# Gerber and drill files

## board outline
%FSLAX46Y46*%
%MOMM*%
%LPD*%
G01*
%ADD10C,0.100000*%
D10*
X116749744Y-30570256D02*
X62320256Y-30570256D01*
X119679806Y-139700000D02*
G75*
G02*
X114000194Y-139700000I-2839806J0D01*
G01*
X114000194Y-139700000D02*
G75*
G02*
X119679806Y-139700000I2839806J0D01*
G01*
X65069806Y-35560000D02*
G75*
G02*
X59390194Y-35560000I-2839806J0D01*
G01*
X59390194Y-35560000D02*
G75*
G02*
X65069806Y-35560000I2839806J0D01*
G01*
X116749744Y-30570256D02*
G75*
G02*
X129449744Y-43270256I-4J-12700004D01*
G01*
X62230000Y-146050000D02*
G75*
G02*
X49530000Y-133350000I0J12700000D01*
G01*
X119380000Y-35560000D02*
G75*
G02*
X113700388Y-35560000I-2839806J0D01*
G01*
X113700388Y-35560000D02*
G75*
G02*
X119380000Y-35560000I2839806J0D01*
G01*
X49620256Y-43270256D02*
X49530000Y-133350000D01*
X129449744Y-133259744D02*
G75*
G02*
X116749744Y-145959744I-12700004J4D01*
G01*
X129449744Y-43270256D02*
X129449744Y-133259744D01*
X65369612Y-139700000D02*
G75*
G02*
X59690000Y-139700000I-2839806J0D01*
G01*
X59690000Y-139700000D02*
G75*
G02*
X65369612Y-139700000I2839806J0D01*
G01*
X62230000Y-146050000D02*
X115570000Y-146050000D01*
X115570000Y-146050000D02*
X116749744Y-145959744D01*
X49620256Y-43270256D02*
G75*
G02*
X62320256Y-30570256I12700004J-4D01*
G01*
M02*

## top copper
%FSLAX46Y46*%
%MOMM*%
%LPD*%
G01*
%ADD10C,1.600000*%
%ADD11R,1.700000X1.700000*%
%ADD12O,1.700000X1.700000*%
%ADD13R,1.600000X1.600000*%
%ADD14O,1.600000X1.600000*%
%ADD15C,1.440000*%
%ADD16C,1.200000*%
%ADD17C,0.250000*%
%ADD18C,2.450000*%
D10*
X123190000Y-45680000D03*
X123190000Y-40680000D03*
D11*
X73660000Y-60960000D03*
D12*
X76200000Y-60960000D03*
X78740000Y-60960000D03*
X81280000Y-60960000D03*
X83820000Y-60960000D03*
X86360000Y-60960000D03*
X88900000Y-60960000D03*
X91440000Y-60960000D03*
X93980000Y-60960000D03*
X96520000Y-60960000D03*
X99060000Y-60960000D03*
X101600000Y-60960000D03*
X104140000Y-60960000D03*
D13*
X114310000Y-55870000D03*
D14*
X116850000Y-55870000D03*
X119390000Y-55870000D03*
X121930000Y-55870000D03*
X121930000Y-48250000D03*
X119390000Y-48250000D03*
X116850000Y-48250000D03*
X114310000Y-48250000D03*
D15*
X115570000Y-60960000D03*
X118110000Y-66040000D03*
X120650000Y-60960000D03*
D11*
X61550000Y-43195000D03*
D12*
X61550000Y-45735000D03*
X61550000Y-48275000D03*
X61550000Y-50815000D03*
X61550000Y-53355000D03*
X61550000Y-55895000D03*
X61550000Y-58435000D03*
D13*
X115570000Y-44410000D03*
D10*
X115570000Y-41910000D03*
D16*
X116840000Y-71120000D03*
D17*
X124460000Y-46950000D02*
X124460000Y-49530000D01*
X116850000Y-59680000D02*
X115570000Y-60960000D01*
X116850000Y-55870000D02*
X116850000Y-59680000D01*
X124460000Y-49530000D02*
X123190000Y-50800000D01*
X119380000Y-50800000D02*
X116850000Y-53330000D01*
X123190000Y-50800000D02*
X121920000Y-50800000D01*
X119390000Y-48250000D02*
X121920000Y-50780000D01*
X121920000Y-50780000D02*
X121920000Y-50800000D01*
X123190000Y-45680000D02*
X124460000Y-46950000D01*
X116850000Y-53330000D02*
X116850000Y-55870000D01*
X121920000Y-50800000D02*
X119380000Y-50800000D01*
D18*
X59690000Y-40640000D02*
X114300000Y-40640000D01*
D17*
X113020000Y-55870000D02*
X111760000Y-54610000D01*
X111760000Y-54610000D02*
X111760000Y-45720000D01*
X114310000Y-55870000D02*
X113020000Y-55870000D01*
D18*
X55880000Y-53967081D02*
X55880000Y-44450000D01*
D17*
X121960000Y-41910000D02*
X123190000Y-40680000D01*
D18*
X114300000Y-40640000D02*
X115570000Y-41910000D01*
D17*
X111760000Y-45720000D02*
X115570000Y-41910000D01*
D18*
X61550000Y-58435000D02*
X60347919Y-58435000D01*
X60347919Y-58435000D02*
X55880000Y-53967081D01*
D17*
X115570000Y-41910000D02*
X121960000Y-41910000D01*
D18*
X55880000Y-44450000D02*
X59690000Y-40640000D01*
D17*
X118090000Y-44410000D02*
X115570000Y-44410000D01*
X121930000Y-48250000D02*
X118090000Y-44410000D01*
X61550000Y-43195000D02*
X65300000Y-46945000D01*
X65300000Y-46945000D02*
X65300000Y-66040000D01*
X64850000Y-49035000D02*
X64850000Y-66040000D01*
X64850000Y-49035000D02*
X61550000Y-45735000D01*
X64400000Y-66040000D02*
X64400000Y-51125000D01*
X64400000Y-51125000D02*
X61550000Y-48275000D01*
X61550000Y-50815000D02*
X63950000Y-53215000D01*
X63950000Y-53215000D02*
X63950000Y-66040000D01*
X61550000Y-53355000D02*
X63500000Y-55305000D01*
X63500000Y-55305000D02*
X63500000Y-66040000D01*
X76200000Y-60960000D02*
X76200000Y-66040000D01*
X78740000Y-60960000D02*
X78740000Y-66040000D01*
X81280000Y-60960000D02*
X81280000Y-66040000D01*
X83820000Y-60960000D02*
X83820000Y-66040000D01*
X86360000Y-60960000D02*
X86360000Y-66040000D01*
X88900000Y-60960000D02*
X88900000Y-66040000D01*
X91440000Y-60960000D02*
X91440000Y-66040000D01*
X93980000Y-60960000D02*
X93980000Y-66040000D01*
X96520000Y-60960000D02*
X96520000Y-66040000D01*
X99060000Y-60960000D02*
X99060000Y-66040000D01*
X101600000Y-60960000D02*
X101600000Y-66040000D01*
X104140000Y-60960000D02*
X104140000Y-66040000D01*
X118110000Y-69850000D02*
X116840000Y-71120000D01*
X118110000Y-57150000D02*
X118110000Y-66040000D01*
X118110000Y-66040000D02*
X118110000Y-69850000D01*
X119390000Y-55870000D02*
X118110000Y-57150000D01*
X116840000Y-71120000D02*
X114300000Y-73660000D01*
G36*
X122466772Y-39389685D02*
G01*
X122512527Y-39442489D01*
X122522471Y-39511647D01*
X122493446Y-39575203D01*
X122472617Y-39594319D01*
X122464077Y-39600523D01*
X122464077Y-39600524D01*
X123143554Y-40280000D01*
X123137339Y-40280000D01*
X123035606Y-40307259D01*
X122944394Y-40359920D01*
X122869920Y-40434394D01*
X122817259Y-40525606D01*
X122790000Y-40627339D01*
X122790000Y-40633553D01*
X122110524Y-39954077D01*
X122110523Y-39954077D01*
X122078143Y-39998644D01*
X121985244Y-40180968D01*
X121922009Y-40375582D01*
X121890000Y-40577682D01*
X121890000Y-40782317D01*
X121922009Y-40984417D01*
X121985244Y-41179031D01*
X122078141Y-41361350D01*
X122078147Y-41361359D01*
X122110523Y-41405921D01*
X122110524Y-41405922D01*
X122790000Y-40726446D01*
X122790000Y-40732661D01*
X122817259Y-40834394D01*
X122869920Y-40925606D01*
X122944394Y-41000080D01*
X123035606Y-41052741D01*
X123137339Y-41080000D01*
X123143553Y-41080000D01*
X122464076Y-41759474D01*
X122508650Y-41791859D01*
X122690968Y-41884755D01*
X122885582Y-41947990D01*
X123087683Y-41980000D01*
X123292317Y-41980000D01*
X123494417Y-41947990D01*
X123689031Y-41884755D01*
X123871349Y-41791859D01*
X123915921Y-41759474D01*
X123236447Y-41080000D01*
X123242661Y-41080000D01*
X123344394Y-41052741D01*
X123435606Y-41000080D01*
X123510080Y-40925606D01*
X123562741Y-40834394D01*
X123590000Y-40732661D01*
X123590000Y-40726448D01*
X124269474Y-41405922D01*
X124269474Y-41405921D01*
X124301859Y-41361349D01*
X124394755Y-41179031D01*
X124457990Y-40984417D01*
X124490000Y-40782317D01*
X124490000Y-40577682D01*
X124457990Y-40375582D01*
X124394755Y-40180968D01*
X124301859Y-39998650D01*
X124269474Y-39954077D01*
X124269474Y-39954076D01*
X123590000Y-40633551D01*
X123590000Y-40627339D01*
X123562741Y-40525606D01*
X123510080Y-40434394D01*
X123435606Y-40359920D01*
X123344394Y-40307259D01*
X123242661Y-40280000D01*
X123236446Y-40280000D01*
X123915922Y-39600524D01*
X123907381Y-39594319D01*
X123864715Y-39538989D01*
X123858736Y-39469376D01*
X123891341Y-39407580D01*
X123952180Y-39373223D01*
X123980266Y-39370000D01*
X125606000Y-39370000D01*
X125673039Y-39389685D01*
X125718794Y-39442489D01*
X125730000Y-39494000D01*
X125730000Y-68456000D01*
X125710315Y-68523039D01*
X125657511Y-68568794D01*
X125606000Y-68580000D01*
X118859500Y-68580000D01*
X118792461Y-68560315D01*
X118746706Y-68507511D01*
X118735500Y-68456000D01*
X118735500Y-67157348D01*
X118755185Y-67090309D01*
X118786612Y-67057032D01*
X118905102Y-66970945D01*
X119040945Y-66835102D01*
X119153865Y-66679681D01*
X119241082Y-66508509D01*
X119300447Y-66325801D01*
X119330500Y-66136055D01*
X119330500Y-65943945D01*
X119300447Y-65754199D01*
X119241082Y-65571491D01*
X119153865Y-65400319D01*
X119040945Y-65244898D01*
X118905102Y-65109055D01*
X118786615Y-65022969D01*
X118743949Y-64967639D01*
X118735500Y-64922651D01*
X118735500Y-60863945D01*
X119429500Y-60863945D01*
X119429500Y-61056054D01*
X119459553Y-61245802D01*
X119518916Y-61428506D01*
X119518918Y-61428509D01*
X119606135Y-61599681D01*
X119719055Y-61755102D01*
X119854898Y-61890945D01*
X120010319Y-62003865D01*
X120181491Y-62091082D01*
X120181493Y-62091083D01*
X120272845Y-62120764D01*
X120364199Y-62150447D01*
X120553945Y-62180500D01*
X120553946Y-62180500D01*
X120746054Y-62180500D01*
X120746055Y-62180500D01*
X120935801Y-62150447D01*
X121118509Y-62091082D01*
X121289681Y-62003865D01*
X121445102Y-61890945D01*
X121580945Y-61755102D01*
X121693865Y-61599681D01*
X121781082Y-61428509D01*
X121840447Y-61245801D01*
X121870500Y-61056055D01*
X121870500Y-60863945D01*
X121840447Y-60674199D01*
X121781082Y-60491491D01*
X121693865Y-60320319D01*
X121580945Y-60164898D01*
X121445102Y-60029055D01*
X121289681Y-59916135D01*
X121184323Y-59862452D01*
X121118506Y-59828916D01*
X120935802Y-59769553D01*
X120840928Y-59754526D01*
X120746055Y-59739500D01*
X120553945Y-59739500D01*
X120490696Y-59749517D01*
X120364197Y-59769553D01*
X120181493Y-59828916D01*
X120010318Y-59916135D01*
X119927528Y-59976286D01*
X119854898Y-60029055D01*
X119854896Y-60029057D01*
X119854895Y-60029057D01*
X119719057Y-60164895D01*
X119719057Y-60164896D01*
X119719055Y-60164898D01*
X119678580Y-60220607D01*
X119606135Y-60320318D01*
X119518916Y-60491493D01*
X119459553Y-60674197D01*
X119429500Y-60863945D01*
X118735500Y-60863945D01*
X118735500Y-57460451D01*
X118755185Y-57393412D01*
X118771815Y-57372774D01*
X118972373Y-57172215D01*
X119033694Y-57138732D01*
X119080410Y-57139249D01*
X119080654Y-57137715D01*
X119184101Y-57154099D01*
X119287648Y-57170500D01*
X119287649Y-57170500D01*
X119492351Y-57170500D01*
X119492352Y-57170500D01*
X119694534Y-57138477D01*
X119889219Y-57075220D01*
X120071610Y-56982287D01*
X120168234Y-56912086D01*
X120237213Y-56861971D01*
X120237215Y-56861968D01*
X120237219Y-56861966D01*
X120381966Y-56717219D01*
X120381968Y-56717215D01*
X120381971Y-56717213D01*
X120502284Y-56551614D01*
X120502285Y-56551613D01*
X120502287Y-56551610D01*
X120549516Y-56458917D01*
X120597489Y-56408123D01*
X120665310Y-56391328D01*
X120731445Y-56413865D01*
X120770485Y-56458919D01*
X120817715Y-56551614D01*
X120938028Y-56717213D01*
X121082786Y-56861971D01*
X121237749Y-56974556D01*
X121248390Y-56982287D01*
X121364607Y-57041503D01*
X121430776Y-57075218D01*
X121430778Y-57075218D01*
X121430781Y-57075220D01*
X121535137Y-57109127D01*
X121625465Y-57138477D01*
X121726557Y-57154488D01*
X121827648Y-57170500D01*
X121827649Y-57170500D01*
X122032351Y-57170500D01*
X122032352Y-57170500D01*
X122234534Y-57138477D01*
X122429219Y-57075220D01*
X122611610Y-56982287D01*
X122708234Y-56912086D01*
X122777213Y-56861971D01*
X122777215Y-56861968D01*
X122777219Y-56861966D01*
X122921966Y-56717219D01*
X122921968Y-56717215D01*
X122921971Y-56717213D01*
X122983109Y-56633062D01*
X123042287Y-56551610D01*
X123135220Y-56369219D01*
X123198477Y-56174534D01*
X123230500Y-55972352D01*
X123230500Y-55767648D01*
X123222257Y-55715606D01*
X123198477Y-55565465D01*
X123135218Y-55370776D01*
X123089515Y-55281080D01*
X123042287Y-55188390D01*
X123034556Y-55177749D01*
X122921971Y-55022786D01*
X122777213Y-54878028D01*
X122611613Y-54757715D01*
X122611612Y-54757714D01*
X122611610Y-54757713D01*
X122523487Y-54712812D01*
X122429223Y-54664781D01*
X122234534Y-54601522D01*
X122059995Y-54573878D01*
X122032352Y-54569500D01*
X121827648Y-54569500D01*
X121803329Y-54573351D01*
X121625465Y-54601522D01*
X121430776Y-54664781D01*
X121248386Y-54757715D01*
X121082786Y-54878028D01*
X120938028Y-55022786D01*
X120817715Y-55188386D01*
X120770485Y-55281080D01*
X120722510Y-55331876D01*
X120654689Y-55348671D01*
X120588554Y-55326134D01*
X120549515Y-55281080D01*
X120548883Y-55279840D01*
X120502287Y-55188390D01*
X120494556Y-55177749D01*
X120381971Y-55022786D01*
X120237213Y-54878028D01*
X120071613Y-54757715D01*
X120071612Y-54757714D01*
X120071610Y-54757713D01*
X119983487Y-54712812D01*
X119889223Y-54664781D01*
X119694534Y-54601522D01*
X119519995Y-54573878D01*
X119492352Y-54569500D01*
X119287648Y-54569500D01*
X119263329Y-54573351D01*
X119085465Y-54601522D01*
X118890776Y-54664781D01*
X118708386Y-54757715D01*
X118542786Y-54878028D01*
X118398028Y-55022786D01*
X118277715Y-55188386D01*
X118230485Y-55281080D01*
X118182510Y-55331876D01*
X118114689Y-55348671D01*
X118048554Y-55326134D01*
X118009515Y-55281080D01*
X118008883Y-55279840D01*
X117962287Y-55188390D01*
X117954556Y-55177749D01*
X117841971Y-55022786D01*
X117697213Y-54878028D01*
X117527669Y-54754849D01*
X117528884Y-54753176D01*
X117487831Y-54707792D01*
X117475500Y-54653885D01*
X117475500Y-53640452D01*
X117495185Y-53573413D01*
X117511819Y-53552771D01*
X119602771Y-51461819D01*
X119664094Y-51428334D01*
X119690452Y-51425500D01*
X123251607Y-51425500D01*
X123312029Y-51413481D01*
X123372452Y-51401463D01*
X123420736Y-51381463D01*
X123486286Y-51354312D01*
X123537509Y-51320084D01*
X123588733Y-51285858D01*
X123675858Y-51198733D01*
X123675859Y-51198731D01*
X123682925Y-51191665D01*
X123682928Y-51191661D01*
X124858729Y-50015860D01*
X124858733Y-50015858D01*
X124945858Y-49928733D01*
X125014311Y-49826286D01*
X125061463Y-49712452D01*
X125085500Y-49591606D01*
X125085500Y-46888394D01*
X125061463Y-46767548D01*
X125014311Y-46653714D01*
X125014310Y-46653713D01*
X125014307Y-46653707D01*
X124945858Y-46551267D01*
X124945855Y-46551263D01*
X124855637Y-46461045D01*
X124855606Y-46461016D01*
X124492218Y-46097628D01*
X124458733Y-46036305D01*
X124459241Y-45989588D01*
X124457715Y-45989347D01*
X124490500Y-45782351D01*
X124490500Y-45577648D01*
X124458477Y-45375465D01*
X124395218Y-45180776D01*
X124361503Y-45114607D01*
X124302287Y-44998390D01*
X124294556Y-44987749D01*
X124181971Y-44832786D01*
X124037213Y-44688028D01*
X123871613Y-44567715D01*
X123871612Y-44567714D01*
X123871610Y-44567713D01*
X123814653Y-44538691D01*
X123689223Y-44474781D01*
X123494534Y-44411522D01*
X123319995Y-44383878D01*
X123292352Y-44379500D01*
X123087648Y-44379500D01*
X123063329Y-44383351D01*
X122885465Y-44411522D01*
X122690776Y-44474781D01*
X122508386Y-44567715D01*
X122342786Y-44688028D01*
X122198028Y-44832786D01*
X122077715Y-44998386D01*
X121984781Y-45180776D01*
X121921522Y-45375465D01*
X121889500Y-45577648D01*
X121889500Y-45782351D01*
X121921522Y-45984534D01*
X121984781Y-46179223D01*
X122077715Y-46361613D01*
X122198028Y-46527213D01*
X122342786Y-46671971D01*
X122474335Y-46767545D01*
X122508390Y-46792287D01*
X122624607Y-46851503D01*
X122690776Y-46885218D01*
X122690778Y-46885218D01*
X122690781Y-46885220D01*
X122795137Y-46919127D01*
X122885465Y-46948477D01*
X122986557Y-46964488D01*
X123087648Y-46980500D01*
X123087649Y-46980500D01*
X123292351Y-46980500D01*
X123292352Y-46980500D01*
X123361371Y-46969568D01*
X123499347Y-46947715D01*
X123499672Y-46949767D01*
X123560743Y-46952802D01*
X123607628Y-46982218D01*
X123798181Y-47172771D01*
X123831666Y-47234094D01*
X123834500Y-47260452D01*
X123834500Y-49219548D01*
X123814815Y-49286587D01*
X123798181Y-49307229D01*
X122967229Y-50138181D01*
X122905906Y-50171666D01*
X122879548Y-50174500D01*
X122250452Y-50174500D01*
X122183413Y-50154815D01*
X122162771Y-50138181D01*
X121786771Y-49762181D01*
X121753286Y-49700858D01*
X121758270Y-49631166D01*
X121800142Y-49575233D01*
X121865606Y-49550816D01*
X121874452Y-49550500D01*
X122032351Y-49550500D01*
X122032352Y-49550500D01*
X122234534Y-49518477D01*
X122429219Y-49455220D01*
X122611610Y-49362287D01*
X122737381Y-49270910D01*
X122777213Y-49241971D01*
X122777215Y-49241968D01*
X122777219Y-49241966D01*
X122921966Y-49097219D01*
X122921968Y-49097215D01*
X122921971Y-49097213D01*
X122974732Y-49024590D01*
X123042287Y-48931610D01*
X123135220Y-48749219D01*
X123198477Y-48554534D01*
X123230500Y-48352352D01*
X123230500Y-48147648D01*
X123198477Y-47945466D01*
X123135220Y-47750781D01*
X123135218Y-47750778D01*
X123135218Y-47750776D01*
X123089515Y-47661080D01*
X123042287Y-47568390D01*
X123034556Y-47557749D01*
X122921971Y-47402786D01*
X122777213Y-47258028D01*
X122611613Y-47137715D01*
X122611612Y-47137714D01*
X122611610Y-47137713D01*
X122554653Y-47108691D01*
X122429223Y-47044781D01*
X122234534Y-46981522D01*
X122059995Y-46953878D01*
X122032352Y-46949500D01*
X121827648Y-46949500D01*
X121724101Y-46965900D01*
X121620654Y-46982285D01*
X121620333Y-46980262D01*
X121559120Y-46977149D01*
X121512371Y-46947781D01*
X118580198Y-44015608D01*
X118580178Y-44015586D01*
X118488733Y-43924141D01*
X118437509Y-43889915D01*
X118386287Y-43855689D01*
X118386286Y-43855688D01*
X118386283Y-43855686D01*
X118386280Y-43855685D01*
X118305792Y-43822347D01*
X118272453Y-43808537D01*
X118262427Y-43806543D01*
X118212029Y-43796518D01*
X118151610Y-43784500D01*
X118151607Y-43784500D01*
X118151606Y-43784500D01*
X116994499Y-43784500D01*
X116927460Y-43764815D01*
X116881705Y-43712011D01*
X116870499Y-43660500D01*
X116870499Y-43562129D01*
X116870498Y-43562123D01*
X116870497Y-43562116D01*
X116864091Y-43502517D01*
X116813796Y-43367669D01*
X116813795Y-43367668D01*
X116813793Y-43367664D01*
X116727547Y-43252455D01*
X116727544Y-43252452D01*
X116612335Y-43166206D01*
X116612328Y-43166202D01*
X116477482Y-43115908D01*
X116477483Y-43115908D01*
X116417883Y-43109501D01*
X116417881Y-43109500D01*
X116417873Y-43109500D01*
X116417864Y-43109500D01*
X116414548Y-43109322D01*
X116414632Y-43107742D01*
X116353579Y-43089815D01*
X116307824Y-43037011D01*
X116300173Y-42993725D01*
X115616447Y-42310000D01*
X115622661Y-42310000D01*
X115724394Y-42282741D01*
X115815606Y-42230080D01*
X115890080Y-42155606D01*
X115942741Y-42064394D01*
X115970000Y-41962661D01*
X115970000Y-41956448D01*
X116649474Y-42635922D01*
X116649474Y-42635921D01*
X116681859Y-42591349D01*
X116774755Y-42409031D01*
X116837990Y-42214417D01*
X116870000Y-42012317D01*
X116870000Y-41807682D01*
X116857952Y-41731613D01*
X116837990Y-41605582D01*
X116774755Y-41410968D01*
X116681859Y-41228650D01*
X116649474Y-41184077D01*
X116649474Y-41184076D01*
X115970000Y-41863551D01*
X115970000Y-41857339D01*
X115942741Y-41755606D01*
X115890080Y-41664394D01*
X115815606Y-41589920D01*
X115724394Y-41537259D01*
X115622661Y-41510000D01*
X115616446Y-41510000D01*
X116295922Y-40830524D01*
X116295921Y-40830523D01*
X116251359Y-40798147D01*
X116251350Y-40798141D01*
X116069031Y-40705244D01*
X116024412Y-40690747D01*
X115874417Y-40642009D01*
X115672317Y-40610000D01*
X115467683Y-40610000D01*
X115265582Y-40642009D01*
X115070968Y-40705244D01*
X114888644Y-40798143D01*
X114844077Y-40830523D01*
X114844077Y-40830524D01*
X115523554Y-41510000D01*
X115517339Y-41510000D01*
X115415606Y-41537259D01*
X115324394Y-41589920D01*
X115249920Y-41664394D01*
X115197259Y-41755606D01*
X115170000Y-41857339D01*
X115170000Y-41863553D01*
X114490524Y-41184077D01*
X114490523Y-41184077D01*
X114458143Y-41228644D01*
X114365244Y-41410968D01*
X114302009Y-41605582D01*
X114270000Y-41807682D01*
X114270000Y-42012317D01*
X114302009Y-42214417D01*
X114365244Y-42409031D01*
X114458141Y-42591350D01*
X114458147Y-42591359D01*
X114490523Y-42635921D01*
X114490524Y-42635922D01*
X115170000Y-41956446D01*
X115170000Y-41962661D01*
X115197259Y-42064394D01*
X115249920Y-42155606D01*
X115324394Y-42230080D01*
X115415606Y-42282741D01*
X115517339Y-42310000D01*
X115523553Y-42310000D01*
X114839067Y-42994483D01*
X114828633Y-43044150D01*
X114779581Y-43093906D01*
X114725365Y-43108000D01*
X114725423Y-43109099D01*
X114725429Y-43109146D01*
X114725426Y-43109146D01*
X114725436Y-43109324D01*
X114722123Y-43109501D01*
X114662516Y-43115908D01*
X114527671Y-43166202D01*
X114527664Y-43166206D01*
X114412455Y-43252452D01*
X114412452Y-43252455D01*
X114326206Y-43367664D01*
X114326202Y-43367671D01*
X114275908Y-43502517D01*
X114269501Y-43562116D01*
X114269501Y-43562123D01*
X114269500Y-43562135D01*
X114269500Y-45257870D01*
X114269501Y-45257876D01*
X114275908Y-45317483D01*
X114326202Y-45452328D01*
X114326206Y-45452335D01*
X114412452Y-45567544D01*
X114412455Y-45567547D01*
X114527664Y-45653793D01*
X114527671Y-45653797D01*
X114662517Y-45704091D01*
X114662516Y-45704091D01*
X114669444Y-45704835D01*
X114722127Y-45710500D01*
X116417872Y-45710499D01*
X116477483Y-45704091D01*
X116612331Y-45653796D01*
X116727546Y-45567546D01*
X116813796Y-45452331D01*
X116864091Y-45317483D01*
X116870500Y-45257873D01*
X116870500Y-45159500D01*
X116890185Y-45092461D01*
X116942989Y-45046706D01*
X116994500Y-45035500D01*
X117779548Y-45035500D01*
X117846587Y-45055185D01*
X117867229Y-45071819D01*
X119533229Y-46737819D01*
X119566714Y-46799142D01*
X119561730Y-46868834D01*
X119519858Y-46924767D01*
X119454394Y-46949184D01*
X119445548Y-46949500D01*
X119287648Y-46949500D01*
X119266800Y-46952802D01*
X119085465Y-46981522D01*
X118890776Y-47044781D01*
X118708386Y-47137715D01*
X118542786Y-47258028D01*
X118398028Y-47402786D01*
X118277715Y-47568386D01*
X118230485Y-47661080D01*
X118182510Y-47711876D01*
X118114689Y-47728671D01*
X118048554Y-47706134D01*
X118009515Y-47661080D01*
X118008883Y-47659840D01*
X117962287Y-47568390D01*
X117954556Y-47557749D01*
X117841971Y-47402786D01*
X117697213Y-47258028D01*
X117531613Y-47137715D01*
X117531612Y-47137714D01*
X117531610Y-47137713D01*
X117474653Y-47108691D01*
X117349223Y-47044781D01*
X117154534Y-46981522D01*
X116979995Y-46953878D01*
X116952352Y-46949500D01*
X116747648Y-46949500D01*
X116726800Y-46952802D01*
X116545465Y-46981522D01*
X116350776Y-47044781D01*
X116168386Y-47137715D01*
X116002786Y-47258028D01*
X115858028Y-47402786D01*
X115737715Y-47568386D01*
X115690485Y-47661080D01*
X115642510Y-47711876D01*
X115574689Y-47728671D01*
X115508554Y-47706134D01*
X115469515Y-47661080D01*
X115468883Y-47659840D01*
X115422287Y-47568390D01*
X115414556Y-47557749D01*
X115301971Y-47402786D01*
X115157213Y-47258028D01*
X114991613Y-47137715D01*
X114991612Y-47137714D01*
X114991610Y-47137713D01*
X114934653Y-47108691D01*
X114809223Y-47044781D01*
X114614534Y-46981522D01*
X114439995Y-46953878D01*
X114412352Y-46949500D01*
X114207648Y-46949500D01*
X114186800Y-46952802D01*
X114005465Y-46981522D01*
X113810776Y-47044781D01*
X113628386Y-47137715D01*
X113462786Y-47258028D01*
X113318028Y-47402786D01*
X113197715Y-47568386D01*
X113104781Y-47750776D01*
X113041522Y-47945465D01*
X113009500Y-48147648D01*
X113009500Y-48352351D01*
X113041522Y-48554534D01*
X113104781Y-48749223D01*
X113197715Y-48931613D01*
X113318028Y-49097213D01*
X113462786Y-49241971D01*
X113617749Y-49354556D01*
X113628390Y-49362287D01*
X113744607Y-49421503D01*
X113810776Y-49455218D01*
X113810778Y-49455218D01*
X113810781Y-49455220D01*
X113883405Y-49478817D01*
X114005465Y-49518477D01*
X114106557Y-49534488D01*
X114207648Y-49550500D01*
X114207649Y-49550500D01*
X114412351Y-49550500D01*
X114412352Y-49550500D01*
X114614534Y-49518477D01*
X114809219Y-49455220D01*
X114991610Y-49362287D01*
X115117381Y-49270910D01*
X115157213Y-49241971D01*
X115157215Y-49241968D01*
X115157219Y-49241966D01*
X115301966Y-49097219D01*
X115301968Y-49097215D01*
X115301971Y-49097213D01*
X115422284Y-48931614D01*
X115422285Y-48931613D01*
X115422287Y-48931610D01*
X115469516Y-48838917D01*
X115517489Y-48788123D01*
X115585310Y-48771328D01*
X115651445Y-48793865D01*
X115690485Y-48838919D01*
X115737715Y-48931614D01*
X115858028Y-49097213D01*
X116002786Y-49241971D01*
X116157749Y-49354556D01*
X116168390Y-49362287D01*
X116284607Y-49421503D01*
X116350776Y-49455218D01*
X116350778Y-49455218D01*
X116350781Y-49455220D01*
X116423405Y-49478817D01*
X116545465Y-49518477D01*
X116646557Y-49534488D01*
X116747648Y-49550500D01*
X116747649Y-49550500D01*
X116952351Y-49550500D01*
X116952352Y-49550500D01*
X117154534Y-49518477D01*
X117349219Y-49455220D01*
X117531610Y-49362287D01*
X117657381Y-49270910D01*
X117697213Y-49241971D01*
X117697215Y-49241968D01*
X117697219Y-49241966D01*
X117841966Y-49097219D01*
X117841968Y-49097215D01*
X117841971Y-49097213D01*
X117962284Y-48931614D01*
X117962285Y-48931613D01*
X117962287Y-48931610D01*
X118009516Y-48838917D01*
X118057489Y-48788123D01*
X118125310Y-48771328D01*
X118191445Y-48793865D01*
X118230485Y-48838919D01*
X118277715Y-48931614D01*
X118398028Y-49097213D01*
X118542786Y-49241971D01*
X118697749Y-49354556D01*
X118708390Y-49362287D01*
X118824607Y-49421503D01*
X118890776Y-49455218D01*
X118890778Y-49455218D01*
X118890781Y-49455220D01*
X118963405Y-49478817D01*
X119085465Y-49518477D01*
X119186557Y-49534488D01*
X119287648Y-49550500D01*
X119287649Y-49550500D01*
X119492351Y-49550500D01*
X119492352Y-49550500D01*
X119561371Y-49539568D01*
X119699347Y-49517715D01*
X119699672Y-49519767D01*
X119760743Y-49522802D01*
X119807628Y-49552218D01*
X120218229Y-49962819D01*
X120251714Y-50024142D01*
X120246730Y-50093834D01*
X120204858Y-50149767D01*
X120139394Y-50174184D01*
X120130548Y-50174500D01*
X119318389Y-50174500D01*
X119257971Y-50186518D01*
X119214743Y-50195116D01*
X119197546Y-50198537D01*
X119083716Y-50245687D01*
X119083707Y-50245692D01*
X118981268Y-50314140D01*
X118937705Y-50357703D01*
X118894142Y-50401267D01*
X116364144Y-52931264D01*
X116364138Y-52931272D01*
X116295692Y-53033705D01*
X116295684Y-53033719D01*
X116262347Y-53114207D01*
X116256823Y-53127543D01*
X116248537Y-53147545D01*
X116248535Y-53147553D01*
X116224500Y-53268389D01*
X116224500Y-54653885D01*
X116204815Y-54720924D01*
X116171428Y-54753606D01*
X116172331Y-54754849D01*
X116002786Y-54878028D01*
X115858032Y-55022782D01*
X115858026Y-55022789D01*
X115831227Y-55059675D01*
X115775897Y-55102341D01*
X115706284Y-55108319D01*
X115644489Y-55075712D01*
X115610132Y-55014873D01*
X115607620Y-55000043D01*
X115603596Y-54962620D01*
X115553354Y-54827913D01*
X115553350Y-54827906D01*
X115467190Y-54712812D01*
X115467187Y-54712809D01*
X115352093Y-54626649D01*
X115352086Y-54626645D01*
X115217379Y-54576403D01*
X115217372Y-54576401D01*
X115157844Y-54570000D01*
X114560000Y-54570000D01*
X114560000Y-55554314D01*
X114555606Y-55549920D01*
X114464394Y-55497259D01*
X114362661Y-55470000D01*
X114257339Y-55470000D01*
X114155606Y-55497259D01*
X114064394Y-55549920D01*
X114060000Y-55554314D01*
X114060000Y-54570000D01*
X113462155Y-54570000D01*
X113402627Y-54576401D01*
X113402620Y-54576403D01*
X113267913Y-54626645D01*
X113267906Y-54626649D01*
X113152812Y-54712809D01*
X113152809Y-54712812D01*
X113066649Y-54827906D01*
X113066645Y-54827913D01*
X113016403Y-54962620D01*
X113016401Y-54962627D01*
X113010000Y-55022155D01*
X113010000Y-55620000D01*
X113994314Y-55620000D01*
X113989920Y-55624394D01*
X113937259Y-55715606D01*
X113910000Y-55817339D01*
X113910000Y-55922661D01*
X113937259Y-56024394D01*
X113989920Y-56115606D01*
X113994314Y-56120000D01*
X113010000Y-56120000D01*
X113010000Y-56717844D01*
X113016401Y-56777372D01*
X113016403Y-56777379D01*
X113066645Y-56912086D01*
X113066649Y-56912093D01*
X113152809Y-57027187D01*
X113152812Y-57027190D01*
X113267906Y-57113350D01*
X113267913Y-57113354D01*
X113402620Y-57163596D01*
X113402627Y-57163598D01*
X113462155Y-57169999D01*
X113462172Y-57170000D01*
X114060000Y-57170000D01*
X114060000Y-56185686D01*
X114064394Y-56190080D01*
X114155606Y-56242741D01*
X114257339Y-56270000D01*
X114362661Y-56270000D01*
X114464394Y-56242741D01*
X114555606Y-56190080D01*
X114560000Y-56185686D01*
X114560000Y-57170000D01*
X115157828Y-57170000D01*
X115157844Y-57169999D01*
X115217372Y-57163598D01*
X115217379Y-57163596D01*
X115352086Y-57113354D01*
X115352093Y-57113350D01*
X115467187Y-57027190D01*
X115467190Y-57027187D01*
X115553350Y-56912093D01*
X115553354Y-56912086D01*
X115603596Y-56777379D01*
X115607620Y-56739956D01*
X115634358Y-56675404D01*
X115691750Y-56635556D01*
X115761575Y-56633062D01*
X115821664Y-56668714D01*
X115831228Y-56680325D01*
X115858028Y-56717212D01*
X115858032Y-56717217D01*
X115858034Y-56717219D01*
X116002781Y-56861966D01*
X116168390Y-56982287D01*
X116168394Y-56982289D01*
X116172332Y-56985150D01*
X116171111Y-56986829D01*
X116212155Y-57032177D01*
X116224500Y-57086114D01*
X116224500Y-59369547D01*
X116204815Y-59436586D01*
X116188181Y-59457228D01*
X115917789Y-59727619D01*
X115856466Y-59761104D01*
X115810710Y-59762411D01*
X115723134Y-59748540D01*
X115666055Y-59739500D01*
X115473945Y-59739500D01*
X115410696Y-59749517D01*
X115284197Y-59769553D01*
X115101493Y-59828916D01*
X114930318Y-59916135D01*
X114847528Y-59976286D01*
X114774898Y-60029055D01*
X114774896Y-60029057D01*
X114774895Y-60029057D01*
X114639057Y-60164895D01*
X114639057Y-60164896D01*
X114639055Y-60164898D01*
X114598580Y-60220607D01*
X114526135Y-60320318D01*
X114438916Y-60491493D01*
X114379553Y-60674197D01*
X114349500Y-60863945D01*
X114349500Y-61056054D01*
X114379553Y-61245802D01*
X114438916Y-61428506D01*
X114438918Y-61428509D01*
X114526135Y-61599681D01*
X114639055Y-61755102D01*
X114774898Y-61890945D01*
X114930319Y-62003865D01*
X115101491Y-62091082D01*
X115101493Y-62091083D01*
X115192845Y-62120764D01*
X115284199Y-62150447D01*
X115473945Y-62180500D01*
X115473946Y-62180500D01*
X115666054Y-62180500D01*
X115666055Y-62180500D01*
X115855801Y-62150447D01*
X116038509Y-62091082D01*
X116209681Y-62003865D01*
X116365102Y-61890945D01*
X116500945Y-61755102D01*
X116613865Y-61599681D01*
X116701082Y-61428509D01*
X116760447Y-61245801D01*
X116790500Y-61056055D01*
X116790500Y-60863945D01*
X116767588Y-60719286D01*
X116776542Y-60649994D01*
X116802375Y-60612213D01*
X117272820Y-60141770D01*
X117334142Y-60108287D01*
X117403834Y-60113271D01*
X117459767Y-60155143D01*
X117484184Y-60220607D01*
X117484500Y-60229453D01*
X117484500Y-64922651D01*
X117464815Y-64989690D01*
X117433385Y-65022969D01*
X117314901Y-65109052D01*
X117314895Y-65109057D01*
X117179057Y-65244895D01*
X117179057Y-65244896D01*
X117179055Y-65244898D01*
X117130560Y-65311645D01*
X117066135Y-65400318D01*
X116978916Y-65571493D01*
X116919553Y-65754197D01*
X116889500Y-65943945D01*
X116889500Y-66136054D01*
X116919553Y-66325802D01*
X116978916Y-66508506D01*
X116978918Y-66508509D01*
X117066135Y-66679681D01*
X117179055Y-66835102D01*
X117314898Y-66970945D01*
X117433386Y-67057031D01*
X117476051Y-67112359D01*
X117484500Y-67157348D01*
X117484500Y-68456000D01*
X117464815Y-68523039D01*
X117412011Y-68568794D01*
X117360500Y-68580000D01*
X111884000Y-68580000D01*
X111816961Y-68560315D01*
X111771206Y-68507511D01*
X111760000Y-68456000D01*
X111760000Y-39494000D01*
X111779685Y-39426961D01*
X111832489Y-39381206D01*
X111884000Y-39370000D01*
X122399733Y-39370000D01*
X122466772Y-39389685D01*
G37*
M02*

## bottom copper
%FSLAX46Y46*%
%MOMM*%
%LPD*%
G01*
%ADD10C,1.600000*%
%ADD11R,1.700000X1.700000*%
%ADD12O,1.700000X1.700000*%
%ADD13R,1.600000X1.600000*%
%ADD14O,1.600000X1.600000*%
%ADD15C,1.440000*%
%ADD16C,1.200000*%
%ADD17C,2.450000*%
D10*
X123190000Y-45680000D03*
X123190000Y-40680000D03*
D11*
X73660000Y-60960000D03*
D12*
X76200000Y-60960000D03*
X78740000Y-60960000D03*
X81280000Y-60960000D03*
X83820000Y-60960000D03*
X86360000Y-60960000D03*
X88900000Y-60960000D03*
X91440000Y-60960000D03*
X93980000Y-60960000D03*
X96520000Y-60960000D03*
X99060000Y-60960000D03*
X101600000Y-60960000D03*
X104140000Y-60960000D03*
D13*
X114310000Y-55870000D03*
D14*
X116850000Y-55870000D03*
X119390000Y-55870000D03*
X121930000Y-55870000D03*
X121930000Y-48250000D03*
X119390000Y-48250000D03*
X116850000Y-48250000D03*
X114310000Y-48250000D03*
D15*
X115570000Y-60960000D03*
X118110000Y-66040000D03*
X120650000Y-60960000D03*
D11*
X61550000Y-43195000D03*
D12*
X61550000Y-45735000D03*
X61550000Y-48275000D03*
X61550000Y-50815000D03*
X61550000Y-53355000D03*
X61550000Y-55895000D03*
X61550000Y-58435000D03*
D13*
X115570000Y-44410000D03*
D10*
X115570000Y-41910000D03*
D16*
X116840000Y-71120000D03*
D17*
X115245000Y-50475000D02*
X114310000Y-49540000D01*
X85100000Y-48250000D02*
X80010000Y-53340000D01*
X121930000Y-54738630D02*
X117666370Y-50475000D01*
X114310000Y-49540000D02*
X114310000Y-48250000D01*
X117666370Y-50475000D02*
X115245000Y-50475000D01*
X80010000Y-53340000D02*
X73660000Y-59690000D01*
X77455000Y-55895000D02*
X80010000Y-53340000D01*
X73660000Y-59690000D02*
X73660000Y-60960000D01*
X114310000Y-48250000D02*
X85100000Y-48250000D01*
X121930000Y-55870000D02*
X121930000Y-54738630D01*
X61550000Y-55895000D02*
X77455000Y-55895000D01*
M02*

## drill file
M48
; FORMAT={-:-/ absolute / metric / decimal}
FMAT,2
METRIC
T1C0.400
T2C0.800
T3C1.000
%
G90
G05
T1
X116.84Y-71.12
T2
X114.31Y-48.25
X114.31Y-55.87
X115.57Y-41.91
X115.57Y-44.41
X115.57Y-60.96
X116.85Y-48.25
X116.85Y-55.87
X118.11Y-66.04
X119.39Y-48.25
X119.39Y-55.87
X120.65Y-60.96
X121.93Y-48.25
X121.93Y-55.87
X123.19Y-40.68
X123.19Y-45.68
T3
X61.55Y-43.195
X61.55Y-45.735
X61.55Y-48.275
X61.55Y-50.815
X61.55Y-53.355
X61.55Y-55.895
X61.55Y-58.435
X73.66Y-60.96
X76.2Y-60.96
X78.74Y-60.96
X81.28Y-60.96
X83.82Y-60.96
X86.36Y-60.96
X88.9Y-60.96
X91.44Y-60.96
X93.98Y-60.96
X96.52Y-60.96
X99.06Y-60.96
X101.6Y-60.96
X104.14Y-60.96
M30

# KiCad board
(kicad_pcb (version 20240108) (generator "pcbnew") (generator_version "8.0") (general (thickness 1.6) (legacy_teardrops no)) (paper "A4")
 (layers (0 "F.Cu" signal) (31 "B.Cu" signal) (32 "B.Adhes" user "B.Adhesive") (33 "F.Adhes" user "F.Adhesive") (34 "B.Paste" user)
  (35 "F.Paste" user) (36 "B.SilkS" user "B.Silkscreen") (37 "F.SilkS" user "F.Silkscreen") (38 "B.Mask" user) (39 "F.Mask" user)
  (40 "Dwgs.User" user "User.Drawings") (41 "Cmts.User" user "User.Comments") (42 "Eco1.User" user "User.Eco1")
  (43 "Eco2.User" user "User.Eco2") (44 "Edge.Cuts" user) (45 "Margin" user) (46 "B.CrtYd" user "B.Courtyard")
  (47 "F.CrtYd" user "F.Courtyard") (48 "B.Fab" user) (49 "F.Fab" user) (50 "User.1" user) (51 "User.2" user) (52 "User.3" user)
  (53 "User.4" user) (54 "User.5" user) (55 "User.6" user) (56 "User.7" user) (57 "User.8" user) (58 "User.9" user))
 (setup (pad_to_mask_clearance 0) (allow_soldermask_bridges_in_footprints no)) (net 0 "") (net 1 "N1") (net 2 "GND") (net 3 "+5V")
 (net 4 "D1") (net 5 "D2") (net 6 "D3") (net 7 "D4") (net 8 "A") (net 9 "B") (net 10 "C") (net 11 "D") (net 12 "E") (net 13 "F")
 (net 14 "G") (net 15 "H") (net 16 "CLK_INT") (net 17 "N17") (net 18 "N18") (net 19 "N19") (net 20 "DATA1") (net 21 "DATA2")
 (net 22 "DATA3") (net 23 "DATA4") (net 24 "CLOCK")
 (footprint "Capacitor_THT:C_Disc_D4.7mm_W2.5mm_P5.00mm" (layer "F.Cu") (at 123.19 45.68 90)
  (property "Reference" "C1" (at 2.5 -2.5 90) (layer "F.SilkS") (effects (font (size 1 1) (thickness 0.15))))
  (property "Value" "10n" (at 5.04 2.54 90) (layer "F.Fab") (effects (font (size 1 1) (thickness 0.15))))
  (pad "1" thru_hole circle (at 0 0 90) (size 1.6 1.6) (drill 0.8) (layers "*.Cu" "*.Mask") (remove_unused_layers no) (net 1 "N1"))
  (pad "2" thru_hole circle (at 5 0 90) (size 1.6 1.6) (drill 0.8) (layers "*.Cu" "*.Mask") (remove_unused_layers no) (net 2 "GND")))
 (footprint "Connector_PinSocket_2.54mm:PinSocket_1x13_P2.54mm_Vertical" (layer "F.Cu") (at 73.66 60.96 90)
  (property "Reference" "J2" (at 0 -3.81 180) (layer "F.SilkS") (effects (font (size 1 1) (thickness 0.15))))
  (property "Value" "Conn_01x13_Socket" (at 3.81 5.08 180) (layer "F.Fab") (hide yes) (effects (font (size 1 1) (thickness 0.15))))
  (pad "1" thru_hole rect (at 0 0 90) (size 1.7 1.7) (drill 1) (layers "*.Cu" "*.Mask") (remove_unused_layers no) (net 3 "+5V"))
  (pad "2" thru_hole oval (at 0 2.54 90) (size 1.7 1.7) (drill 1) (layers "*.Cu" "*.Mask") (remove_unused_layers no) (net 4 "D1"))
  (pad "3" thru_hole oval (at 0 5.08 90) (size 1.7 1.7) (drill 1) (layers "*.Cu" "*.Mask") (remove_unused_layers no) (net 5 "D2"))
  (pad "4" thru_hole oval (at 0 7.62 90) (size 1.7 1.7) (drill 1) (layers "*.Cu" "*.Mask") (remove_unused_layers no) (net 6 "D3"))
  (pad "5" thru_hole oval (at 0 10.16 90) (size 1.7 1.7) (drill 1) (layers "*.Cu" "*.Mask") (remove_unused_layers no) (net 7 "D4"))
  (pad "6" thru_hole oval (at 0 12.7 90) (size 1.7 1.7) (drill 1) (layers "*.Cu" "*.Mask") (remove_unused_layers no) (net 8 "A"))
  (pad "7" thru_hole oval (at 0 15.24 90) (size 1.7 1.7) (drill 1) (layers "*.Cu" "*.Mask") (remove_unused_layers no) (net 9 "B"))
  (pad "8" thru_hole oval (at 0 17.78 90) (size 1.7 1.7) (drill 1) (layers "*.Cu" "*.Mask") (remove_unused_layers no) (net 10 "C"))
  (pad "9" thru_hole oval (at 0 20.32 90) (size 1.7 1.7) (drill 1) (layers "*.Cu" "*.Mask") (remove_unused_layers no) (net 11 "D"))
  (pad "10" thru_hole oval (at 0 22.86 90) (size 1.7 1.7) (drill 1) (layers "*.Cu" "*.Mask") (remove_unused_layers no) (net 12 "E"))
  (pad "11" thru_hole oval (at 0 25.4 90) (size 1.7 1.7) (drill 1) (layers "*.Cu" "*.Mask") (remove_unused_layers no) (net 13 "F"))
  (pad "12" thru_hole oval (at 0 27.94 90) (size 1.7 1.7) (drill 1) (layers "*.Cu" "*.Mask") (remove_unused_layers no) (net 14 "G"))
  (pad "13" thru_hole oval (at 0 30.48 90) (size 1.7 1.7) (drill 1) (layers "*.Cu" "*.Mask") (remove_unused_layers no) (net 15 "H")))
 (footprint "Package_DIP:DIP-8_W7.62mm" (layer "F.Cu") (at 114.31 55.87 90)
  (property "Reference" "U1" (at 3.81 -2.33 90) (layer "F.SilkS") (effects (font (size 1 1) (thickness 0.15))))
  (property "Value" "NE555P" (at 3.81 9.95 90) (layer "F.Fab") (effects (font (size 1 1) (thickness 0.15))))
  (pad "1" thru_hole rect (at 0 0 90) (size 1.6 1.6) (drill 0.8) (layers "*.Cu" "*.Mask") (remove_unused_layers no) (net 2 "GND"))
  (pad "2" thru_hole oval (at 0 2.54 90) (size 1.6 1.6) (drill 0.8) (layers "*.Cu" "*.Mask") (remove_unused_layers no) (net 1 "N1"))
  (pad "3" thru_hole oval (at 0 5.08 90) (size 1.6 1.6) (drill 0.8) (layers "*.Cu" "*.Mask") (remove_unused_layers no) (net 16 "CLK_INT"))
  (pad "4" thru_hole oval (at 0 7.62 90) (size 1.6 1.6) (drill 0.8) (layers "*.Cu" "*.Mask") (remove_unused_layers no) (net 3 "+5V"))
  (pad "5" thru_hole oval (at 7.62 7.62 90) (size 1.6 1.6) (drill 0.8) (layers "*.Cu" "*.Mask") (remove_unused_layers no) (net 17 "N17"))
  (pad "6" thru_hole oval (at 7.62 5.08 90) (size 1.6 1.6) (drill 0.8) (layers "*.Cu" "*.Mask") (remove_unused_layers no) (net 1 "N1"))
  (pad "7" thru_hole oval (at 7.62 2.54 90) (size 1.6 1.6) (drill 0.8) (layers "*.Cu" "*.Mask") (remove_unused_layers no) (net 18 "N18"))
  (pad "8" thru_hole oval (at 7.62 0 90) (size 1.6 1.6) (drill 0.8) (layers "*.Cu" "*.Mask") (remove_unused_layers no) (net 3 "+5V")))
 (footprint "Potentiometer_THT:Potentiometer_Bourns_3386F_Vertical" (layer "F.Cu") (at 115.57 60.96 -90)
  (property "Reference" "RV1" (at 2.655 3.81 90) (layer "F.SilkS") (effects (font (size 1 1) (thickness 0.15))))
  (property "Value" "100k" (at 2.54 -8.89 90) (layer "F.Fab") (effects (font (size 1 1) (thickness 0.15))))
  (pad "1" thru_hole circle (at 0 0 270) (size 1.44 1.44) (drill 0.8) (layers "*.Cu" "*.Mask") (remove_unused_layers no) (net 1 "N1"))
  (pad "2" thru_hole circle (at 5.08 -2.54 270) (size 1.44 1.44) (drill 0.8) (layers "*.Cu" "*.Mask") (remove_unused_layers no)
   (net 16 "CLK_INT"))
  (pad "3" thru_hole circle (at 0 -5.08 270) (size 1.44 1.44) (drill 0.8) (layers "*.Cu" "*.Mask") (remove_unused_layers no) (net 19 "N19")))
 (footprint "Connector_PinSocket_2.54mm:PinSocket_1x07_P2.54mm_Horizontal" (layer "F.Cu") (at 61.55 43.195)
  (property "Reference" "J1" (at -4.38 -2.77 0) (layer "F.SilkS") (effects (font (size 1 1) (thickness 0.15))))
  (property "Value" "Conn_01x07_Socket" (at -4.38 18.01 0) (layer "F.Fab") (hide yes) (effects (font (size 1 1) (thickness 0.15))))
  (pad "1" thru_hole rect (at 0 0) (size 1.7 1.7) (drill 1) (layers "*.Cu" "*.Mask") (remove_unused_layers no) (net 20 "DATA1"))
  (pad "2" thru_hole oval (at 0 2.54) (size 1.7 1.7) (drill 1) (layers "*.Cu" "*.Mask") (remove_unused_layers no) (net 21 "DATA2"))
  (pad "3" thru_hole oval (at 0 5.08) (size 1.7 1.7) (drill 1) (layers "*.Cu" "*.Mask") (remove_unused_layers no) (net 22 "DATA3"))
  (pad "4" thru_hole oval (at 0 7.62) (size 1.7 1.7) (drill 1) (layers "*.Cu" "*.Mask") (remove_unused_layers no) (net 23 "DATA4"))
  (pad "5" thru_hole oval (at 0 10.16) (size 1.7 1.7) (drill 1) (layers "*.Cu" "*.Mask") (remove_unused_layers no) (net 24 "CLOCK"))
  (pad "6" thru_hole oval (at 0 12.7) (size 1.7 1.7) (drill 1) (layers "*.Cu" "*.Mask") (remove_unused_layers no) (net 3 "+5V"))
  (pad "7" thru_hole oval (at 0 15.24) (size 1.7 1.7) (drill 1) (layers "*.Cu" "*.Mask") (remove_unused_layers no) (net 2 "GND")))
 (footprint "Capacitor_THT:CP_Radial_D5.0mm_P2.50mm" (layer "F.Cu") (at 115.57 44.41 90)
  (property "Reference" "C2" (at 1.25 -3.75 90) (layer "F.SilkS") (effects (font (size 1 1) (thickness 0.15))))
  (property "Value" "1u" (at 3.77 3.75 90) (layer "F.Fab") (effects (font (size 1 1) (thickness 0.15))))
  (pad "1" thru_hole rect (at 0 0 90) (size 1.6 1.6) (drill 0.8) (layers "*.Cu" "*.Mask") (remove_unused_layers no) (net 17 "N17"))
  (pad "2" thru_hole circle (at 2.5 0 90) (size 1.6 1.6) (drill 0.8) (layers "*.Cu" "*.Mask") (remove_unused_layers no) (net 2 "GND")))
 (gr_line (start 116.749744 30.570256) (end 62.320256 30.570256) (stroke (width 0.1) (type default)) (layer "Edge.Cuts"))
 (gr_circle (center 116.84 139.7) (end 119.38 140.97) (stroke (width 0.1) (type default)) (fill none) (layer "Edge.Cuts"))
 (gr_circle (center 62.23 35.56) (end 64.77 36.83) (stroke (width 0.1) (type default)) (fill none) (layer "Edge.Cuts"))
 (gr_arc (start 116.749744 30.570256) (mid 125.73 34.29) (end 129.449744 43.270256) (stroke (width 0.1) (type default)) (layer "Edge.Cuts"))
 (gr_arc (start 62.23 146.05) (mid 53.249744 142.330256) (end 49.53 133.35) (stroke (width 0.1) (type default)) (layer "Edge.Cuts"))
 (gr_circle (center 116.540194 35.56) (end 119.080194 36.83) (stroke (width 0.1) (type default)) (fill none) (layer "Edge.Cuts"))
 (gr_line (start 49.620256 43.270256) (end 49.53 133.35) (stroke (width 0.1) (type default)) (layer "Edge.Cuts"))
 (gr_arc (start 129.449744 133.259744) (mid 125.73 142.24) (end 116.749744 145.959744) (stroke (width 0.1) (type default))
  (layer "Edge.Cuts"))
 (gr_line (start 129.449744 43.270256) (end 129.449744 133.259744) (stroke (width 0.1) (type default)) (layer "Edge.Cuts"))
 (gr_circle (center 62.529806 139.7) (end 65.069806 140.97) (stroke (width 0.1) (type default)) (fill none) (layer "Edge.Cuts"))
 (gr_line (start 62.23 146.05) (end 115.57 146.05) (stroke (width 0.1) (type default)) (layer "Edge.Cuts"))
 (gr_line (start 115.57 146.05) (end 116.749744 145.959744) (stroke (width 0.1) (type default)) (layer "Edge.Cuts"))
 (gr_arc (start 49.620256 43.270256) (mid 53.34 34.29) (end 62.320256 30.570256) (stroke (width 0.1) (type default)) (layer "Edge.Cuts"))
 (segment (start 124.46 46.95) (end 124.46 49.53) (width 0.25) (layer "F.Cu") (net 1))
 (segment (start 116.85 59.68) (end 115.57 60.96) (width 0.25) (layer "F.Cu") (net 1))
 (segment (start 116.85 55.87) (end 116.85 59.68) (width 0.25) (layer "F.Cu") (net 1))
 (segment (start 124.46 49.53) (end 123.19 50.8) (width 0.25) (layer "F.Cu") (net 1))
 (segment (start 119.38 50.8) (end 116.85 53.33) (width 0.25) (layer "F.Cu") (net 1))
 (segment (start 123.19 50.8) (end 121.92 50.8) (width 0.25) (layer "F.Cu") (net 1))
 (segment (start 119.39 48.25) (end 121.92 50.78) (width 0.25) (layer "F.Cu") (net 1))
 (segment (start 121.92 50.78) (end 121.92 50.8) (width 0.25) (layer "F.Cu") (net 1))
 (segment (start 123.19 45.68) (end 124.46 46.95) (width 0.25) (layer "F.Cu") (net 1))
 (segment (start 116.85 53.33) (end 116.85 55.87) (width 0.25) (layer "F.Cu") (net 1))
 (segment (start 121.92 50.8) (end 119.38 50.8) (width 0.25) (layer "F.Cu") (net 1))
 (segment (start 59.69 40.64) (end 114.3 40.64) (width 2.45) (layer "F.Cu") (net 2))
 (segment (start 113.02 55.87) (end 111.76 54.61) (width 0.25) (layer "F.Cu") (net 2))
 (segment (start 111.76 54.61) (end 111.76 45.72) (width 0.25) (layer "F.Cu") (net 2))
 (segment (start 114.31 55.87) (end 113.02 55.87) (width 0.25) (layer "F.Cu") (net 2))
 (segment (start 55.88 53.967081) (end 55.88 44.45) (width 2.45) (layer "F.Cu") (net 2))
 (segment (start 121.96 41.91) (end 123.19 40.68) (width 0.25) (layer "F.Cu") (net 2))
 (segment (start 114.3 40.64) (end 115.57 41.91) (width 2.45) (layer "F.Cu") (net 2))
 (segment (start 111.76 45.72) (end 115.57 41.91) (width 0.25) (layer "F.Cu") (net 2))
 (segment (start 61.55 58.435) (end 60.347919 58.435) (width 2.45) (layer "F.Cu") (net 2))
 (segment (start 60.347919 58.435) (end 55.88 53.967081) (width 2.45) (layer "F.Cu") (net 2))
 (segment (start 115.57 41.91) (end 121.96 41.91) (width 0.25) (layer "F.Cu") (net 2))
 (segment (start 55.88 44.45) (end 59.69 40.64) (width 2.45) (layer "F.Cu") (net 2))
 (segment (start 118.09 44.41) (end 115.57 44.41) (width 0.25) (layer "F.Cu") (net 17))
 (segment (start 121.93 48.25) (end 118.09 44.41) (width 0.25) (layer "F.Cu") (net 17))
 (segment (start 61.55 43.195) (end 65.3 46.945) (width 0.25) (layer "F.Cu") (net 20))
 (segment (start 65.3 46.945) (end 65.3 66.04) (width 0.25) (layer "F.Cu") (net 20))
 (segment (start 64.85 49.035) (end 64.85 66.04) (width 0.25) (layer "F.Cu") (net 21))
 (segment (start 64.85 49.035) (end 61.55 45.735) (width 0.25) (layer "F.Cu") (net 21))
 (segment (start 64.4 66.04) (end 64.4 51.125) (width 0.25) (layer "F.Cu") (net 22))
 (segment (start 64.4 51.125) (end 61.55 48.275) (width 0.25) (layer "F.Cu") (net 22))
 (segment (start 61.55 50.815) (end 63.95 53.215) (width 0.25) (layer "F.Cu") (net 23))
 (segment (start 63.95 53.215) (end 63.95 66.04) (width 0.25) (layer "F.Cu") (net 23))
 (segment (start 61.55 53.355) (end 63.5 55.305) (width 0.25) (layer "F.Cu") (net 24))
 (segment (start 63.5 55.305) (end 63.5 66.04) (width 0.25) (layer "F.Cu") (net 24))
 (segment (start 115.245 50.475) (end 114.31 49.54) (width 2.45) (layer "B.Cu") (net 3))
 (segment (start 85.1 48.25) (end 80.01 53.34) (width 2.45) (layer "B.Cu") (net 3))
 (segment (start 121.93 54.73863) (end 117.66637 50.475) (width 2.45) (layer "B.Cu") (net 3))
 (segment (start 114.31 49.54) (end 114.31 48.25) (width 2.45) (layer "B.Cu") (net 3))
 (segment (start 117.66637 50.475) (end 115.245 50.475) (width 2.45) (layer "B.Cu") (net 3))
 (segment (start 80.01 53.34) (end 73.66 59.69) (width 2.45) (layer "B.Cu") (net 3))
 (segment (start 77.455 55.895) (end 80.01 53.34) (width 2.45) (layer "B.Cu") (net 3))
 (segment (start 73.66 59.69) (end 73.66 60.96) (width 2.45) (layer "B.Cu") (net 3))
 (segment (start 114.31 48.25) (end 85.1 48.25) (width 2.45) (layer "B.Cu") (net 3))
 (segment (start 121.93 55.87) (end 121.93 54.73863) (width 2.45) (layer "B.Cu") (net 3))
 (segment (start 61.55 55.895) (end 77.455 55.895) (width 2.45) (layer "B.Cu") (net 3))
 (segment (start 76.2 60.96) (end 76.2 66.04) (width 0.25) (layer "F.Cu") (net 4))
 (segment (start 78.74 60.96) (end 78.74 66.04) (width 0.25) (layer "F.Cu") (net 5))
 (segment (start 81.28 60.96) (end 81.28 66.04) (width 0.25) (layer "F.Cu") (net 6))
 (segment (start 83.82 60.96) (end 83.82 66.04) (width 0.25) (layer "F.Cu") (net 7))
 (segment (start 86.36 60.96) (end 86.36 66.04) (width 0.25) (layer "F.Cu") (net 8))
 (segment (start 88.9 60.96) (end 88.9 66.04) (width 0.25) (layer "F.Cu") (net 9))
 (segment (start 91.44 60.96) (end 91.44 66.04) (width 0.25) (layer "F.Cu") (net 10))
 (segment (start 93.98 60.96) (end 93.98 66.04) (width 0.25) (layer "F.Cu") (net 11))
 (segment (start 96.52 60.96) (end 96.52 66.04) (width 0.25) (layer "F.Cu") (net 12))
 (segment (start 99.06 60.96) (end 99.06 66.04) (width 0.25) (layer "F.Cu") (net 13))
 (segment (start 101.6 60.96) (end 101.6 66.04) (width 0.25) (layer "F.Cu") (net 14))
 (segment (start 104.14 60.96) (end 104.14 66.04) (width 0.25) (layer "F.Cu") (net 15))
 (segment (start 118.11 69.85) (end 116.84 71.12) (width 0.25) (layer "F.Cu") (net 16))
 (segment (start 118.11 57.15) (end 118.11 66.04) (width 0.25) (layer "F.Cu") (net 16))
 (segment (start 118.11 66.04) (end 118.11 69.85) (width 0.25) (layer "F.Cu") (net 16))
 (segment (start 119.39 55.87) (end 118.11 57.15) (width 0.25) (layer "F.Cu") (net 16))
 (segment (start 116.84 71.12) (end 114.3 73.66) (width 0.25) (layer "F.Cu") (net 16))
 (via (at 116.84 71.12) (size 1.2) (drill 0.4) (layers "F.Cu" "B.Cu") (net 16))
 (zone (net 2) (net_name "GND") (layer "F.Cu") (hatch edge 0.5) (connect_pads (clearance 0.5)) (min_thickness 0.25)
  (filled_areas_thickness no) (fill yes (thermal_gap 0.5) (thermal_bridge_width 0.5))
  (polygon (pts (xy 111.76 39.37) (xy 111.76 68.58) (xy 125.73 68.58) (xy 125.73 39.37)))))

